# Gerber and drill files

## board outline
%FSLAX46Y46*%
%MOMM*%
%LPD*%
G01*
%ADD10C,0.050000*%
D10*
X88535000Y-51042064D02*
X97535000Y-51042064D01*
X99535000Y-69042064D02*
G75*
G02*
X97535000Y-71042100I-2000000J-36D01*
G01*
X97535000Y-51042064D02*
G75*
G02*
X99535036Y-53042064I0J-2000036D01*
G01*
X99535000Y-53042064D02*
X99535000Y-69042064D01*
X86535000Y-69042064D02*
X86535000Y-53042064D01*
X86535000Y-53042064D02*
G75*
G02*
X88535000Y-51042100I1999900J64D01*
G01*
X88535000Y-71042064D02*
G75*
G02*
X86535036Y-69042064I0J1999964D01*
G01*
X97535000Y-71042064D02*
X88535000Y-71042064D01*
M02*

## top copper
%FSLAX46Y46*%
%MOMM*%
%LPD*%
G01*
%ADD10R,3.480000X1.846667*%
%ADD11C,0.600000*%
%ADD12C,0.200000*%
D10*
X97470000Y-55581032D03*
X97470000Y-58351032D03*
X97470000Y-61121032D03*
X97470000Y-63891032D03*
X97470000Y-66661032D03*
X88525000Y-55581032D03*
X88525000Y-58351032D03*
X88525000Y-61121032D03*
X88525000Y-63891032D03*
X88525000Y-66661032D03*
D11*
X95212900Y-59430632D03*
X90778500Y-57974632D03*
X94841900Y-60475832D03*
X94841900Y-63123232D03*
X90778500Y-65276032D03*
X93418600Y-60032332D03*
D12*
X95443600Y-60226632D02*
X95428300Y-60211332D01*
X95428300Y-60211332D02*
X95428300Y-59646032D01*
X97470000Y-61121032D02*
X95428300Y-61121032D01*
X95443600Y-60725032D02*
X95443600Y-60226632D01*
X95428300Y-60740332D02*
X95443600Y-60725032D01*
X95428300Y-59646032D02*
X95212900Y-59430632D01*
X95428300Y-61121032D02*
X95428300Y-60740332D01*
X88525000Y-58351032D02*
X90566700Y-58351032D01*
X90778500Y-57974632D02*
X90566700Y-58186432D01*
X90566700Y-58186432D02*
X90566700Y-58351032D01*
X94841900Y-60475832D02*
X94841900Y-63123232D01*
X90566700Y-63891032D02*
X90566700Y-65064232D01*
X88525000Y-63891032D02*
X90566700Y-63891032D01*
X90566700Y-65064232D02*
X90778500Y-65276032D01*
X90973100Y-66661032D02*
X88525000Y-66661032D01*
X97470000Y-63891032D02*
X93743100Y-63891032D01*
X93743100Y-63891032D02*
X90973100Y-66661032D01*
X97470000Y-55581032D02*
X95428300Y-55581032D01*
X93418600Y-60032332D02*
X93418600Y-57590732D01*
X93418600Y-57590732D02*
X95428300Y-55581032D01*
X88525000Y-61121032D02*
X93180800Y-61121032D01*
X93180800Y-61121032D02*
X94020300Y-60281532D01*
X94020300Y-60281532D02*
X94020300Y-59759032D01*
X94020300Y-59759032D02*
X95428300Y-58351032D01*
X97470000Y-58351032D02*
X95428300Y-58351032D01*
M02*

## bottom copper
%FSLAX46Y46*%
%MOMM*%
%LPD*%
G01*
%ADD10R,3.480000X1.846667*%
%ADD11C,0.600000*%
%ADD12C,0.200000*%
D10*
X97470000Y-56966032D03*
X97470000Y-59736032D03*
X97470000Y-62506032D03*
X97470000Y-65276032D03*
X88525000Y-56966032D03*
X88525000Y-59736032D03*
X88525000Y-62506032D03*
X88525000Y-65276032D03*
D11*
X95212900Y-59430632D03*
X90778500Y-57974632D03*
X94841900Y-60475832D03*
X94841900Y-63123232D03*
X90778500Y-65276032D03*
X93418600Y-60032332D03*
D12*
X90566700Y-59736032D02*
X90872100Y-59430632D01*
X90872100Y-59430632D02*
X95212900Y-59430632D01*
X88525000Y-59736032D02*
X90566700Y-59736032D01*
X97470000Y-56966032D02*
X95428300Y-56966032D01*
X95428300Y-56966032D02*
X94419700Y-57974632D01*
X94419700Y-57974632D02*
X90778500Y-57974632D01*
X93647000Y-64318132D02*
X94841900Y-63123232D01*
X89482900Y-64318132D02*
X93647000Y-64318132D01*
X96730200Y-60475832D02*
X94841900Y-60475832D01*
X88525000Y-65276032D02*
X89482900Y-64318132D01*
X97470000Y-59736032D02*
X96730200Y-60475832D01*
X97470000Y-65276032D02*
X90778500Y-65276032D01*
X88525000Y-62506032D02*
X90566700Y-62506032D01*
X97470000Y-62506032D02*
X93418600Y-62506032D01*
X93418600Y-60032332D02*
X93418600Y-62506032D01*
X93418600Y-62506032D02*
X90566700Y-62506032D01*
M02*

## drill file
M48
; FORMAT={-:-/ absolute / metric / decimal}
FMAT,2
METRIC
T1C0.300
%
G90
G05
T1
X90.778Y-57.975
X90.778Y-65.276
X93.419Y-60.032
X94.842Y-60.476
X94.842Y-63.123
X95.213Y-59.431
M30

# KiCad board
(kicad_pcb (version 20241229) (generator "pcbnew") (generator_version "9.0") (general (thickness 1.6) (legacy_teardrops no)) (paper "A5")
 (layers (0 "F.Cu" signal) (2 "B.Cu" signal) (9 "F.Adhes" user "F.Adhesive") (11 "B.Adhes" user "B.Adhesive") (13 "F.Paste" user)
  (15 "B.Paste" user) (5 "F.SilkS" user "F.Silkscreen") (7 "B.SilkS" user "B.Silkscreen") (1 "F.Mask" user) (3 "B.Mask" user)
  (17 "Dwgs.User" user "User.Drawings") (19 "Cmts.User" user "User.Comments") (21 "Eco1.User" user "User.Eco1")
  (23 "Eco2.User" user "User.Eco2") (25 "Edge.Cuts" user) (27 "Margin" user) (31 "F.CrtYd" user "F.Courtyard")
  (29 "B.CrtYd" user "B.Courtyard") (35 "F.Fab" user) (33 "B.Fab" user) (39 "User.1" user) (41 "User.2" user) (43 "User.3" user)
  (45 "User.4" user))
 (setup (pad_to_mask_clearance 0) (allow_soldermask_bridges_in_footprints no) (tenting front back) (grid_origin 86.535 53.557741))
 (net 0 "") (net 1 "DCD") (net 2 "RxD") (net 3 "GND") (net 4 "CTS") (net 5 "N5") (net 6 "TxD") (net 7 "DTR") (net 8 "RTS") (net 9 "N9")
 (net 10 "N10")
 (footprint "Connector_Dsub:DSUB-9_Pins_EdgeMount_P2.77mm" (layer "F.Cu") (at 97.47 61.121032 90)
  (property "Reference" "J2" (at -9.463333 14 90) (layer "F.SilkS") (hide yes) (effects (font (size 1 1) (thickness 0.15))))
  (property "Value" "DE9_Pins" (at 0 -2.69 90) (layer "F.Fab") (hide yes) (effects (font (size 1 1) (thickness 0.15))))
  (pad "1" smd rect (at 5.54 0 90) (size 1.846667 3.48) (layers "F.Cu" "F.Mask" "F.Paste") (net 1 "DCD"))
  (pad "2" smd rect (at 2.77 0 90) (size 1.846667 3.48) (layers "F.Cu" "F.Mask" "F.Paste") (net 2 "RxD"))
  (pad "3" smd rect (at 0 0 90) (size 1.846667 3.48) (layers "F.Cu" "F.Mask" "F.Paste") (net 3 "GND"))
  (pad "4" smd rect (at -2.77 0 90) (size 1.846667 3.48) (layers "F.Cu" "F.Mask" "F.Paste") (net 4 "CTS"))
  (pad "5" smd rect (at -5.54 0 90) (size 1.846667 3.48) (layers "F.Cu" "F.Mask" "F.Paste") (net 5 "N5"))
  (pad "6" smd rect (at 4.155 0 90) (size 1.846667 3.48) (layers "B.Cu" "B.Mask" "B.Paste") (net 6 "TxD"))
  (pad "7" smd rect (at 1.385 0 90) (size 1.846667 3.48) (layers "B.Cu" "B.Mask" "B.Paste") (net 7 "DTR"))
  (pad "8" smd rect (at -1.385 0 90) (size 1.846667 3.48) (layers "B.Cu" "B.Mask" "B.Paste") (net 1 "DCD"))
  (pad "9" smd rect (at -4.155 0 90) (size 1.846667 3.48) (layers "B.Cu" "B.Mask" "B.Paste") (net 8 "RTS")))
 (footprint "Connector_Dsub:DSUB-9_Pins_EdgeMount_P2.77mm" (layer "F.Cu") (at 88.525 61.121032 -90)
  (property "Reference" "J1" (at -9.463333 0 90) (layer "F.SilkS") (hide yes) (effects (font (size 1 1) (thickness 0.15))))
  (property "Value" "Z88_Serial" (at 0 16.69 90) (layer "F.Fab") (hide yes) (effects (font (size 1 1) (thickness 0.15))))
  (pad "1" smd rect (at -5.54 0 270) (size 1.846667 3.48) (layers "F.Cu" "F.Mask" "F.Paste") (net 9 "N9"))
  (pad "2" smd rect (at -2.77 0 270) (size 1.846667 3.48) (layers "F.Cu" "F.Mask" "F.Paste") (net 6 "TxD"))
  (pad "3" smd rect (at 0 0 270) (size 1.846667 3.48) (layers "F.Cu" "F.Mask" "F.Paste") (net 2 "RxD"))
  (pad "4" smd rect (at 2.77 0 270) (size 1.846667 3.48) (layers "F.Cu" "F.Mask" "F.Paste") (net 8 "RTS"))
  (pad "5" smd rect (at 5.54 0 270) (size 1.846667 3.48) (layers "F.Cu" "F.Mask" "F.Paste") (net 4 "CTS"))
  (pad "6" smd rect (at -4.155 0 270) (size 1.846667 3.48) (layers "B.Cu" "B.Mask" "B.Paste") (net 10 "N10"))
  (pad "7" smd rect (at -1.385 0 270) (size 1.846667 3.48) (layers "B.Cu" "B.Mask" "B.Paste") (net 3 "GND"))
  (pad "8" smd rect (at 1.385 0 270) (size 1.846667 3.48) (layers "B.Cu" "B.Mask" "B.Paste") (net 1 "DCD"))
  (pad "9" smd rect (at 4.155 0 270) (size 1.846667 3.48) (layers "B.Cu" "B.Mask" "B.Paste") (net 7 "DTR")))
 (gr_line (start 88.535 51.042064) (end 97.535 51.042064) (stroke (width 0.05) (type default)) (layer "Edge.Cuts"))
 (gr_arc (start 99.535 69.042064) (mid 98.949214 70.456278) (end 97.535 71.042064) (stroke (width 0.05) (type default)) (layer "Edge.Cuts"))
 (gr_arc (start 97.535 51.042064) (mid 98.949214 51.62785) (end 99.535 53.042064) (stroke (width 0.05) (type default)) (layer "Edge.Cuts"))
 (gr_line (start 99.535 53.042064) (end 99.535 69.042064) (stroke (width 0.05) (type default)) (layer "Edge.Cuts"))
 (gr_line (start 86.535 69.042064) (end 86.535 53.042064) (stroke (width 0.05) (type default)) (layer "Edge.Cuts"))
 (gr_arc (start 86.535 53.042064) (mid 87.120775 51.62783) (end 88.535 51.042064) (stroke (width 0.05) (type default)) (layer "Edge.Cuts"))
 (gr_arc (start 88.535 71.042064) (mid 87.120775 70.45628) (end 86.535 69.042064) (stroke (width 0.05) (type default)) (layer "Edge.Cuts"))
 (gr_line (start 97.535 71.042064) (end 88.535 71.042064) (stroke (width 0.05) (type default)) (layer "Edge.Cuts"))
 (segment (start 95.4436 60.226632) (end 95.4283 60.211332) (width 0.2) (layer "F.Cu") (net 3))
 (segment (start 95.4283 60.211332) (end 95.4283 59.646032) (width 0.2) (layer "F.Cu") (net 3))
 (segment (start 97.47 61.121032) (end 95.4283 61.121032) (width 0.2) (layer "F.Cu") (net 3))
 (segment (start 95.4436 60.725032) (end 95.4436 60.226632) (width 0.2) (layer "F.Cu") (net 3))
 (segment (start 95.4283 60.740332) (end 95.4436 60.725032) (width 0.2) (layer "F.Cu") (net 3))
 (segment (start 95.4283 59.646032) (end 95.2129 59.430632) (width 0.2) (layer "F.Cu") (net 3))
 (segment (start 95.4283 61.121032) (end 95.4283 60.740332) (width 0.2) (layer "F.Cu") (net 3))
 (via (at 95.2129 59.430632) (size 0.6) (drill 0.3) (layers "F.Cu" "B.Cu") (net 3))
 (segment (start 90.5667 59.736032) (end 90.8721 59.430632) (width 0.2) (layer "B.Cu") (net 3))
 (segment (start 90.8721 59.430632) (end 95.2129 59.430632) (width 0.2) (layer "B.Cu") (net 3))
 (segment (start 88.525 59.736032) (end 90.5667 59.736032) (width 0.2) (layer "B.Cu") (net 3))
 (segment (start 88.525 58.351032) (end 90.5667 58.351032) (width 0.2) (layer "F.Cu") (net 6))
 (segment (start 90.7785 57.974632) (end 90.5667 58.186432) (width 0.2) (layer "F.Cu") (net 6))
 (segment (start 90.5667 58.186432) (end 90.5667 58.351032) (width 0.2) (layer "F.Cu") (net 6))
 (via (at 90.7785 57.974632) (size 0.6) (drill 0.3) (layers "F.Cu" "B.Cu") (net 6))
 (segment (start 97.47 56.966032) (end 95.4283 56.966032) (width 0.2) (layer "B.Cu") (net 6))
 (segment (start 95.4283 56.966032) (end 94.4197 57.974632) (width 0.2) (layer "B.Cu") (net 6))
 (segment (start 94.4197 57.974632) (end 90.7785 57.974632) (width 0.2) (layer "B.Cu") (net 6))
 (segment (start 94.8419 60.475832) (end 94.8419 63.123232) (width 0.2) (layer "F.Cu") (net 7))
 (via (at 94.8419 60.475832) (size 0.6) (drill 0.3) (layers "F.Cu" "B.Cu") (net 7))
 (via (at 94.8419 63.123232) (size 0.6) (drill 0.3) (layers "F.Cu" "B.Cu") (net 7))
 (segment (start 93.647 64.318132) (end 94.8419 63.123232) (width 0.2) (layer "B.Cu") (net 7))
 (segment (start 89.4829 64.318132) (end 93.647 64.318132) (width 0.2) (layer "B.Cu") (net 7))
 (segment (start 96.7302 60.475832) (end 94.8419 60.475832) (width 0.2) (layer "B.Cu") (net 7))
 (segment (start 88.525 65.276032) (end 89.4829 64.318132) (width 0.2) (layer "B.Cu") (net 7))
 (segment (start 97.47 59.736032) (end 96.7302 60.475832) (width 0.2) (layer "B.Cu") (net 7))
 (segment (start 90.5667 63.891032) (end 90.5667 65.064232) (width 0.2) (layer "F.Cu") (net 8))
 (segment (start 88.525 63.891032) (end 90.5667 63.891032) (width 0.2) (layer "F.Cu") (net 8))
 (segment (start 90.5667 65.064232) (end 90.7785 65.276032) (width 0.2) (layer "F.Cu") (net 8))
 (via (at 90.7785 65.276032) (size 0.6) (drill 0.3) (layers "F.Cu" "B.Cu") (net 8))
 (segment (start 97.47 65.276032) (end 90.7785 65.276032) (width 0.2) (layer "B.Cu") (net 8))
 (segment (start 90.9731 66.661032) (end 88.525 66.661032) (width 0.2) (layer "F.Cu") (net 4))
 (segment (start 97.47 63.891032) (end 93.7431 63.891032) (width 0.2) (layer "F.Cu") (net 4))
 (segment (start 93.7431 63.891032) (end 90.9731 66.661032) (width 0.2) (layer "F.Cu") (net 4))
 (segment (start 97.47 55.581032) (end 95.4283 55.581032) (width 0.2) (layer "F.Cu") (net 1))
 (segment (start 93.4186 60.032332) (end 93.4186 57.590732) (width 0.2) (layer "F.Cu") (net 1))
 (segment (start 93.4186 57.590732) (end 95.4283 55.581032) (width 0.2) (layer "F.Cu") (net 1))
 (via (at 93.4186 60.032332) (size 0.6) (drill 0.3) (layers "F.Cu" "B.Cu") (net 1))
 (segment (start 88.525 62.506032) (end 90.5667 62.506032) (width 0.2) (layer "B.Cu") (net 1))
 (segment (start 97.47 62.506032) (end 93.4186 62.506032) (width 0.2) (layer "B.Cu") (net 1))
 (segment (start 93.4186 60.032332) (end 93.4186 62.506032) (width 0.2) (layer "B.Cu") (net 1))
 (segment (start 93.4186 62.506032) (end 90.5667 62.506032) (width 0.2) (layer "B.Cu") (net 1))
 (segment (start 88.525 61.121032) (end 93.1808 61.121032) (width 0.2) (layer "F.Cu") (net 2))
 (segment (start 93.1808 61.121032) (end 94.0203 60.281532) (width 0.2) (layer "F.Cu") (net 2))
 (segment (start 94.0203 60.281532) (end 94.0203 59.759032) (width 0.2) (layer "F.Cu") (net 2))
 (segment (start 94.0203 59.759032) (end 95.4283 58.351032) (width 0.2) (layer "F.Cu") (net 2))
 (segment (start 97.47 58.351032) (end 95.4283 58.351032) (width 0.2) (layer "F.Cu") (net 2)))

